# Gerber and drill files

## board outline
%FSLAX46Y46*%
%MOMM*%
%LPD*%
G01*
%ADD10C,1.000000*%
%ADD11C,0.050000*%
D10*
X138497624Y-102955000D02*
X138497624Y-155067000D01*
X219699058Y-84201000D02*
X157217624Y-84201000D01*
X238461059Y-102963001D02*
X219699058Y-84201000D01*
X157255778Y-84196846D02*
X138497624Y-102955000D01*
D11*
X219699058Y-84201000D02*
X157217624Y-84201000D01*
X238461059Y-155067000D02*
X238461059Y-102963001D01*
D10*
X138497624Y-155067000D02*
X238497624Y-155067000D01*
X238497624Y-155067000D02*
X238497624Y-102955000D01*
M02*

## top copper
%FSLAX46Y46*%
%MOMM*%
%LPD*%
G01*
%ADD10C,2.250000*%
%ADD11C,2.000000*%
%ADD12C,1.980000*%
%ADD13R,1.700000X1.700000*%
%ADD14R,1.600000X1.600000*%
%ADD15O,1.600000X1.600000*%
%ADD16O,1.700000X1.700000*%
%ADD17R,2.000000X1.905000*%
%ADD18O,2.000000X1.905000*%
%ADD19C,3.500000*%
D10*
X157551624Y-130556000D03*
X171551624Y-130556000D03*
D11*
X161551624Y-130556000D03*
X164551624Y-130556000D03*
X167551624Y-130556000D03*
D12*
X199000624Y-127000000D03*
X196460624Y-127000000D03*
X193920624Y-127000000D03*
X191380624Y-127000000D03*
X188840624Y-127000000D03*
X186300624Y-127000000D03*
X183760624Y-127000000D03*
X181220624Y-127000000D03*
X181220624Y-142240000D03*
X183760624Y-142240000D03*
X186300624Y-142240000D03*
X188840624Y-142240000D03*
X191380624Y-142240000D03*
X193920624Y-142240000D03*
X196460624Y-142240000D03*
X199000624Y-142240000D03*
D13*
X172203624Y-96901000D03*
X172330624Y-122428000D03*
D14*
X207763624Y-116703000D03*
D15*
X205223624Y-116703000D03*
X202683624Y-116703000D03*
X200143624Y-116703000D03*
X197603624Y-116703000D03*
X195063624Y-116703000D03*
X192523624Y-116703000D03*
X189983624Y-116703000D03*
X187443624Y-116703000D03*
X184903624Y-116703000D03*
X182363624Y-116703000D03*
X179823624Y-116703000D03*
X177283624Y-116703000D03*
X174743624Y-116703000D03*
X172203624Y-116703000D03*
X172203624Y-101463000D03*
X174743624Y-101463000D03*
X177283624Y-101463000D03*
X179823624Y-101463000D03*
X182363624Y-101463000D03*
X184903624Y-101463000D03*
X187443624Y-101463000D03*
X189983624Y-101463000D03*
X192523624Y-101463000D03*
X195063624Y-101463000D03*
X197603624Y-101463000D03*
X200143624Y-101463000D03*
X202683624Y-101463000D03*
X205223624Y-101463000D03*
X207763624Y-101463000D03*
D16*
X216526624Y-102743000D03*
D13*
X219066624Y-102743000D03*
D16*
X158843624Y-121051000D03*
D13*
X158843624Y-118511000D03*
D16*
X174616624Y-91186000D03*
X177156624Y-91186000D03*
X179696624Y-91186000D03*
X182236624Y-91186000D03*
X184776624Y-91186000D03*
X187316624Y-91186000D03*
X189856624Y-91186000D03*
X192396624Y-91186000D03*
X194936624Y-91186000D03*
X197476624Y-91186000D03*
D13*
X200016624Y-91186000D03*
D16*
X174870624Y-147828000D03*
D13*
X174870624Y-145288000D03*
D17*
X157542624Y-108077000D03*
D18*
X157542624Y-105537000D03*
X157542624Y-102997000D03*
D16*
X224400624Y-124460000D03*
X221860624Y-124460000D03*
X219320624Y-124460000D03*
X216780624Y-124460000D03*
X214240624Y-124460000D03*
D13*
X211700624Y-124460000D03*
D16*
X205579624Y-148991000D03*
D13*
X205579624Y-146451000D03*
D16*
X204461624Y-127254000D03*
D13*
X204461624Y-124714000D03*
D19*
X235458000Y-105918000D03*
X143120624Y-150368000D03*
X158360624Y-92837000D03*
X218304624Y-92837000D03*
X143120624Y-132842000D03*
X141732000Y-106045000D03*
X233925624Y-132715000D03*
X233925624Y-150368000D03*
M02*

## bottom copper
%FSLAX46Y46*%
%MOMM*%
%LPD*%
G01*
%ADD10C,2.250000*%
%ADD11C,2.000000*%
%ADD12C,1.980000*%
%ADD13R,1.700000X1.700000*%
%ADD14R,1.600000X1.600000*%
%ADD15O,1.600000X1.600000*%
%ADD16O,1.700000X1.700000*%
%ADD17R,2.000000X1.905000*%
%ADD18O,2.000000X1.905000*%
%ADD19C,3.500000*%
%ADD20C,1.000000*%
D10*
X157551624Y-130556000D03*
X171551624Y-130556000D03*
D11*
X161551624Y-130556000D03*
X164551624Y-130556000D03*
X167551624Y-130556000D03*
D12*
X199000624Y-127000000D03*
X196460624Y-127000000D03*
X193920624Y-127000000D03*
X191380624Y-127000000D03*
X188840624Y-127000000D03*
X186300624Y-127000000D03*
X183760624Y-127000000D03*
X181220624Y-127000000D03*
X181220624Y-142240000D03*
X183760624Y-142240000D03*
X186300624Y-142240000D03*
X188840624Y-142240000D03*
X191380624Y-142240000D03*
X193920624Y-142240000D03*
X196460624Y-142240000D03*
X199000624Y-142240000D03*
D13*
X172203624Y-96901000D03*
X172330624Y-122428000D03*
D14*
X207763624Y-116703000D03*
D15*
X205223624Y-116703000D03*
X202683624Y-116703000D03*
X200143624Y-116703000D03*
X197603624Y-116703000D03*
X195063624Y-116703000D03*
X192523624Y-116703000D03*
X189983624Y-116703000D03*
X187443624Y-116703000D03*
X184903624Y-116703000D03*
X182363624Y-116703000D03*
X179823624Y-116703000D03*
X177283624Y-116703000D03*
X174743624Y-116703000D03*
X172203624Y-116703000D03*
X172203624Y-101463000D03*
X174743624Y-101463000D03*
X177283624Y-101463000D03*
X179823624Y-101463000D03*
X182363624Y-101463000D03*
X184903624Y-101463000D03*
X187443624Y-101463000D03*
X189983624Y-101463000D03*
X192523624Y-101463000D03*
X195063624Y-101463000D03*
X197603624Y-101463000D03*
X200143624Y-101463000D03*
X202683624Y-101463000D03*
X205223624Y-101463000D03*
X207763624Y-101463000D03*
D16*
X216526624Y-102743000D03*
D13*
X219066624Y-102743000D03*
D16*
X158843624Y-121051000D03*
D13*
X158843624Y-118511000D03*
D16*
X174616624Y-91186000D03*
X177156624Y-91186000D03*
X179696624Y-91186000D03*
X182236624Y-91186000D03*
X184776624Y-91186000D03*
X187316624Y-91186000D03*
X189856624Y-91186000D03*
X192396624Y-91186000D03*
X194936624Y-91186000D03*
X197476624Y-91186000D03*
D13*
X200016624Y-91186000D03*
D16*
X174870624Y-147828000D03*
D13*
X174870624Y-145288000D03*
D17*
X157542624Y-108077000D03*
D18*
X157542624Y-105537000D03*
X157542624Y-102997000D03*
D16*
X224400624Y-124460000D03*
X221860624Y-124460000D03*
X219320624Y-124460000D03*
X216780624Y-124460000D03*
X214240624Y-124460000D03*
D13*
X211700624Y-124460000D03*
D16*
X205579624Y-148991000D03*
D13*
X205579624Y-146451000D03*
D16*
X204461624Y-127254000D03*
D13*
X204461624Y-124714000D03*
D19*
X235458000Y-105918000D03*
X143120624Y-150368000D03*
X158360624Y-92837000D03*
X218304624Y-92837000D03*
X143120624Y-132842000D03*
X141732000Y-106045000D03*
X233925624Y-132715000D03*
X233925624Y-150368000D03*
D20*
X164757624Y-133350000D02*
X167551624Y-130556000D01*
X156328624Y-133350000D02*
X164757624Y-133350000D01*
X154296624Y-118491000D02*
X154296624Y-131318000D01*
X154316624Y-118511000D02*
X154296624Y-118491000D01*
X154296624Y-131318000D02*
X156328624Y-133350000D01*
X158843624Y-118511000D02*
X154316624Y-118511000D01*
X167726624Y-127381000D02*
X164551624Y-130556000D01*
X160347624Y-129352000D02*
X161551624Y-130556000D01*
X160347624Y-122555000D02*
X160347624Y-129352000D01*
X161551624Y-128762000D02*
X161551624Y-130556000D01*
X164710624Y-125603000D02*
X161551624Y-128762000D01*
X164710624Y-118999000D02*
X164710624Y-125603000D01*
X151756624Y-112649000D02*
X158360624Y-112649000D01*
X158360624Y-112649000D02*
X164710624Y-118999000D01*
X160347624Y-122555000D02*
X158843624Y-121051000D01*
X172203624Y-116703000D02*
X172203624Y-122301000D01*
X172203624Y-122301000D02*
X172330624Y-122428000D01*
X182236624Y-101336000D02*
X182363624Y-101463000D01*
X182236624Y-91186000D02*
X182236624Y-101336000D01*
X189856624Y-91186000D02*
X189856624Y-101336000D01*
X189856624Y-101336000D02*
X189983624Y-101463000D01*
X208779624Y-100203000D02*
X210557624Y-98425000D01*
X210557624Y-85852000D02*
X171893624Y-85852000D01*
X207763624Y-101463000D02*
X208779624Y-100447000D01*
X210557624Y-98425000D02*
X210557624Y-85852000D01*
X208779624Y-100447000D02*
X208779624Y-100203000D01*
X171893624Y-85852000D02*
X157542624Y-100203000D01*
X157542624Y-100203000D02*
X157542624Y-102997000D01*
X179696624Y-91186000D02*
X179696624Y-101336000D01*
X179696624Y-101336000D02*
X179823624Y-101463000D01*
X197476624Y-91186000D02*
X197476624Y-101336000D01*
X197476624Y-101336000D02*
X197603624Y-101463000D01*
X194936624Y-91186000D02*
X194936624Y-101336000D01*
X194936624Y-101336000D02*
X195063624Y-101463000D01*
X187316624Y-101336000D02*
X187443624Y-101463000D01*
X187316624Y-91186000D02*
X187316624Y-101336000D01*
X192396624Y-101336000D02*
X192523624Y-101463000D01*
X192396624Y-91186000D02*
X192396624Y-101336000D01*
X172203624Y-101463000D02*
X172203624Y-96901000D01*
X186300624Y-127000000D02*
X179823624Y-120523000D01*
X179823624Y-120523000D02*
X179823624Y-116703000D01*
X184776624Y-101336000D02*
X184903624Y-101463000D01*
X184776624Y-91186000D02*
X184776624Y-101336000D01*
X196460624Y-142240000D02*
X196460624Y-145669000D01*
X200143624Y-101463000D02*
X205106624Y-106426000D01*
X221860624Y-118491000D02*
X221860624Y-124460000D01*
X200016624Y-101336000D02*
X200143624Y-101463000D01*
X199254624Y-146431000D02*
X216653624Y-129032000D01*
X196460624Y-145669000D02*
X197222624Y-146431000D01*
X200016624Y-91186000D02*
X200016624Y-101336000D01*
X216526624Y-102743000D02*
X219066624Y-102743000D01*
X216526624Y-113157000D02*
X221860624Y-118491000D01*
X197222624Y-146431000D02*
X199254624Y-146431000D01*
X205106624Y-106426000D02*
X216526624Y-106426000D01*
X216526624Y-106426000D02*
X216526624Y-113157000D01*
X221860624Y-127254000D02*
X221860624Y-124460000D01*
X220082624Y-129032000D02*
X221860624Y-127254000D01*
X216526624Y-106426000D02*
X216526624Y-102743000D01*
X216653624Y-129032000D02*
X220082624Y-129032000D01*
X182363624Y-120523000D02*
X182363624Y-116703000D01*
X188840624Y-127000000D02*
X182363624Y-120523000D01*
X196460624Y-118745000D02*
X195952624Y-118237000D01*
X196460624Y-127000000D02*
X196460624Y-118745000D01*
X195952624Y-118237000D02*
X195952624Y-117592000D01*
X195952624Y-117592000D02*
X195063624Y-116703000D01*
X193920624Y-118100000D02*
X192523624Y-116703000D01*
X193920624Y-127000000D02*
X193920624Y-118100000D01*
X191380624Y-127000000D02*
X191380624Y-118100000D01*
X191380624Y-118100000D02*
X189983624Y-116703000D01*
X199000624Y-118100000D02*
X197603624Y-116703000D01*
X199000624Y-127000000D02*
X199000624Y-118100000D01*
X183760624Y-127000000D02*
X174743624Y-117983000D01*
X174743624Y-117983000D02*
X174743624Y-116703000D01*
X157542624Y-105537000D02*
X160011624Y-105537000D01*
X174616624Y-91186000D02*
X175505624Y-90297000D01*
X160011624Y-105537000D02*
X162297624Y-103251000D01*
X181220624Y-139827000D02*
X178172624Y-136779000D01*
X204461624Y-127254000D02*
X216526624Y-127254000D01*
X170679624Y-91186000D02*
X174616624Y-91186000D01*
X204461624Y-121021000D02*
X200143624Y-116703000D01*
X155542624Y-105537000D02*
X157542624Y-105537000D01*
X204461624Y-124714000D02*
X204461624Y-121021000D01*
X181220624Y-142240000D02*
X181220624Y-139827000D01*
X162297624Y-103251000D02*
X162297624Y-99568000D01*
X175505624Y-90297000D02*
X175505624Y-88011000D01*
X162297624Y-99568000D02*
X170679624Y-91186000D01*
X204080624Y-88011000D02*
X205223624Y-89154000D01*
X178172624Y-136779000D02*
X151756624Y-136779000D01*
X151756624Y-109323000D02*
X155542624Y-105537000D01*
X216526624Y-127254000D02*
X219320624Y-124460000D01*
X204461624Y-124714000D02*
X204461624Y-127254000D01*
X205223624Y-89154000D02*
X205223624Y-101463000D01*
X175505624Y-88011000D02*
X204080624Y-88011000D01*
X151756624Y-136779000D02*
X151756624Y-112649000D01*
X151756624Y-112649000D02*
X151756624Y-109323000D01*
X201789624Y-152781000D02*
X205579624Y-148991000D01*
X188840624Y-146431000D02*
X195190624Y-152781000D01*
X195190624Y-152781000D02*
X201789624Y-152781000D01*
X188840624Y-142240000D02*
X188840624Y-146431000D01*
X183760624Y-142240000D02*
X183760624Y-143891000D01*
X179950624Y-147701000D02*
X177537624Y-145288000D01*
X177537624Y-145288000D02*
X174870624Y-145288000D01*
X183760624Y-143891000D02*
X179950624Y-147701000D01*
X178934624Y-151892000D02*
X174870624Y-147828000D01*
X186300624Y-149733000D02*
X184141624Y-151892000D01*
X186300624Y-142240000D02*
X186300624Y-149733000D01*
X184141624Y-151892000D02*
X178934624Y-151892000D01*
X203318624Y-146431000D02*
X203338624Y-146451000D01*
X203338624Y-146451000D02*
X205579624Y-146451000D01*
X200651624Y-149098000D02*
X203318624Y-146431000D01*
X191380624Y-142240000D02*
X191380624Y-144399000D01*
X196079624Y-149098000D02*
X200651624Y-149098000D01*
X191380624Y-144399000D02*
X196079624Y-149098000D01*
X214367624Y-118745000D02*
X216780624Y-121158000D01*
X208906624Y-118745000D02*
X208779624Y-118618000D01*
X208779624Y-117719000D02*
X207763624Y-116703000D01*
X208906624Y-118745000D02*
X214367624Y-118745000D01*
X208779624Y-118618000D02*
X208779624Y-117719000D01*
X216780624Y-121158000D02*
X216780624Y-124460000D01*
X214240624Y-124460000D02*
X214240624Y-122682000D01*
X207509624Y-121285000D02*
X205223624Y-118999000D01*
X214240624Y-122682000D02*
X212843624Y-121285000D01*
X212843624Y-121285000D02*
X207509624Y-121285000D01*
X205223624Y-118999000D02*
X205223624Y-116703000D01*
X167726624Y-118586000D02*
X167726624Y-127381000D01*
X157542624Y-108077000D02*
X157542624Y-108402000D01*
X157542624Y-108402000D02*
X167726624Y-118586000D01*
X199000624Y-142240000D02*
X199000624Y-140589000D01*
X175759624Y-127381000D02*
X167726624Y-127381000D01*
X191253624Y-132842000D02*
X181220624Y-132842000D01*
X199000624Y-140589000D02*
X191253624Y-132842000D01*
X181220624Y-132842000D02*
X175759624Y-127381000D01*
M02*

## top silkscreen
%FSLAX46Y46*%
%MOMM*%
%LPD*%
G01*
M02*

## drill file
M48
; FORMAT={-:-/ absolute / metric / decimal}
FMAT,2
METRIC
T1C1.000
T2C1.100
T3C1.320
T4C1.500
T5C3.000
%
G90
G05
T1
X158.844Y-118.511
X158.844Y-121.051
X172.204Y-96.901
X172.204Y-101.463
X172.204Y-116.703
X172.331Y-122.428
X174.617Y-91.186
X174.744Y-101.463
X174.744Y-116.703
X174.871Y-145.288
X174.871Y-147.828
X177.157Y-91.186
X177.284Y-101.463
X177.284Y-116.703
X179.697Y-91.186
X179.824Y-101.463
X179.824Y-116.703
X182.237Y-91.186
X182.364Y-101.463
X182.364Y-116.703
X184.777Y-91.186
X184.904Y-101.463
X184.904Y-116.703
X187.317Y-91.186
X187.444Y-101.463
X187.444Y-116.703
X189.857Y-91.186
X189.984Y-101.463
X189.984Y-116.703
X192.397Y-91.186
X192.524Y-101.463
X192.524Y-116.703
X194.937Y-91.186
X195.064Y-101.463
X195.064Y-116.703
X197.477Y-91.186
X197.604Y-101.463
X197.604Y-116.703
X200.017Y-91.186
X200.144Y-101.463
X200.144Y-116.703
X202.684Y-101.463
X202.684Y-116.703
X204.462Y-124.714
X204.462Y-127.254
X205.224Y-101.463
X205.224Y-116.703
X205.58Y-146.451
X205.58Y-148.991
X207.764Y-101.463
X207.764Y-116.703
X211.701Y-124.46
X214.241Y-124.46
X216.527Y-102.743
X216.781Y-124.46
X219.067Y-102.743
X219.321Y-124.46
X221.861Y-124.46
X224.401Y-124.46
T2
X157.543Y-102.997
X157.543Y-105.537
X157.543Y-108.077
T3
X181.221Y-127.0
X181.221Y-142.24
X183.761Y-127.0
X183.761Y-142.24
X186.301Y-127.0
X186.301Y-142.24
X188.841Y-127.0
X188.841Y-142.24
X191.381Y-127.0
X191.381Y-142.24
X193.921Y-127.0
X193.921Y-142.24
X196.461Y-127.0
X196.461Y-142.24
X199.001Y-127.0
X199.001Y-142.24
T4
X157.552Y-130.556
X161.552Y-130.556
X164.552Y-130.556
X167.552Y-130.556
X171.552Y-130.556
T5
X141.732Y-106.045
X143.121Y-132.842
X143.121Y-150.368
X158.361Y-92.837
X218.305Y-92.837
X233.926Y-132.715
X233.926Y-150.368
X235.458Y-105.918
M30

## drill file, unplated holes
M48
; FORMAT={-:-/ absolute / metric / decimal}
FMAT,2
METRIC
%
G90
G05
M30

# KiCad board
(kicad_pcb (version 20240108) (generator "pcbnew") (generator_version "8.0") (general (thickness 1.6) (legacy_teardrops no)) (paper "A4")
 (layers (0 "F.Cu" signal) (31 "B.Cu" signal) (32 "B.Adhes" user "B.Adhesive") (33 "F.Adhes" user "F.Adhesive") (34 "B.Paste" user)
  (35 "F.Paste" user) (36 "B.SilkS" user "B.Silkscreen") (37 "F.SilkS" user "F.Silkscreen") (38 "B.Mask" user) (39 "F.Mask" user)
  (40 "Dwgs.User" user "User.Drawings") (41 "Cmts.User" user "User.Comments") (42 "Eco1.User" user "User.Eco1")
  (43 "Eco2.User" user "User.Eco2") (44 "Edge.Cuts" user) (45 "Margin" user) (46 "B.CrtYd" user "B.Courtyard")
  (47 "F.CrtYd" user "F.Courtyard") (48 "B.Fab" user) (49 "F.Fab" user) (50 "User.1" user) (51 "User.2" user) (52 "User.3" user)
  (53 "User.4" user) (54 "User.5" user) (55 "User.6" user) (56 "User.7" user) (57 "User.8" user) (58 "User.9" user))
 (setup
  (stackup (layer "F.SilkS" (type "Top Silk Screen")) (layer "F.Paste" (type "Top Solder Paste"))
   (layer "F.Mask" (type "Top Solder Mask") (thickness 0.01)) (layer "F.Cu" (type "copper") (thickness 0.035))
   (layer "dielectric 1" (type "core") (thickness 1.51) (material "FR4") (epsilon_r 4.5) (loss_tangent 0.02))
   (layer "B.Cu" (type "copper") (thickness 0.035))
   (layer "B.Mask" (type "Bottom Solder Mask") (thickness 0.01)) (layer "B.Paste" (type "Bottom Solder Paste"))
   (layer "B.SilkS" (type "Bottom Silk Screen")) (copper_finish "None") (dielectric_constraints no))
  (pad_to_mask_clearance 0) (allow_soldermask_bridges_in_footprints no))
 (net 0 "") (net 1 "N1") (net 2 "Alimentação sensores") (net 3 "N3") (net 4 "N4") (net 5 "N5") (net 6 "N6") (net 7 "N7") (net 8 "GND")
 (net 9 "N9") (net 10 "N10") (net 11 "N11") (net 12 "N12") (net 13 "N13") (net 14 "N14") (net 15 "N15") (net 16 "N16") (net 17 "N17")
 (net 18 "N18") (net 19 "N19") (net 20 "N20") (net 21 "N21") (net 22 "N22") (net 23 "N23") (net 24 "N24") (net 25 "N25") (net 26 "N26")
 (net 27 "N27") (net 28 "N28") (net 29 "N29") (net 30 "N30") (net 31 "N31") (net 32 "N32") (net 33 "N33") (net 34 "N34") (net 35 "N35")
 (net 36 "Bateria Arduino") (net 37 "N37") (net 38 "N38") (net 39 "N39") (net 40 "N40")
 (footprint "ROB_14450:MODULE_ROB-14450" (layer "B.Cu") (at 190.110624 134.62 90)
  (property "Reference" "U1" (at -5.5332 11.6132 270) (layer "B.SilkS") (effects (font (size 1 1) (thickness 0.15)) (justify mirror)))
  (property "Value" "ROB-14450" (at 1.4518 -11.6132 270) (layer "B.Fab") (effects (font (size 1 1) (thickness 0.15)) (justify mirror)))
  (pad "1" thru_hole circle (at -7.62 8.89 90) (size 1.98 1.98) (drill 1.32) (layers "*.Cu" "*.Mask") (remove_unused_layers no) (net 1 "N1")
   (solder_mask_margin 0.102))
  (pad "2" thru_hole circle (at -7.62 6.35 90) (size 1.98 1.98) (drill 1.32) (layers "*.Cu" "*.Mask") (remove_unused_layers no)
   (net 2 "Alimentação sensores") (solder_mask_margin 0.102))
  (pad "3" thru_hole circle (at -7.62 3.81 90) (size 1.98 1.98) (drill 1.32) (layers "*.Cu" "*.Mask") (remove_unused_layers no) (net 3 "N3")
   (solder_mask_margin 0.102))
  (pad "4" thru_hole circle (at -7.62 1.27 90) (size 1.98 1.98) (drill 1.32) (layers "*.Cu" "*.Mask") (remove_unused_layers no) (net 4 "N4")
   (solder_mask_margin 0.102))
  (pad "5" thru_hole circle (at -7.62 -1.27 90) (size 1.98 1.98) (drill 1.32) (layers "*.Cu" "*.Mask") (remove_unused_layers no)
   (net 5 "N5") (solder_mask_margin 0.102))
  (pad "6" thru_hole circle (at -7.62 -3.81 90) (size 1.98 1.98) (drill 1.32) (layers "*.Cu" "*.Mask") (remove_unused_layers no)
   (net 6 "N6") (solder_mask_margin 0.102))
  (pad "7" thru_hole circle (at -7.62 -6.35 90) (size 1.98 1.98) (drill 1.32) (layers "*.Cu" "*.Mask") (remove_unused_layers no)
   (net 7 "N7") (solder_mask_margin 0.102))
  (pad "8" thru_hole circle (at -7.62 -8.89 90) (size 1.98 1.98) (drill 1.32) (layers "*.Cu" "*.Mask") (remove_unused_layers no)
   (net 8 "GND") (solder_mask_margin 0.102))
  (pad "9" thru_hole circle (at 7.62 -8.89 90) (size 1.98 1.98) (drill 1.32) (layers "*.Cu" "*.Mask") (remove_unused_layers no) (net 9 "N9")
   (solder_mask_margin 0.102))
  (pad "10" thru_hole circle (at 7.62 -6.35 90) (size 1.98 1.98) (drill 1.32) (layers "*.Cu" "*.Mask") (remove_unused_layers no)
   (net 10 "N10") (solder_mask_margin 0.102))
  (pad "11" thru_hole circle (at 7.62 -3.81 90) (size 1.98 1.98) (drill 1.32) (layers "*.Cu" "*.Mask") (remove_unused_layers no)
   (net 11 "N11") (solder_mask_margin 0.102))
  (pad "12" thru_hole circle (at 7.62 -1.27 90) (size 1.98 1.98) (drill 1.32) (layers "*.Cu" "*.Mask") (remove_unused_layers no)
   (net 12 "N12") (solder_mask_margin 0.102))
  (pad "13" thru_hole circle (at 7.62 1.27 90) (size 1.98 1.98) (drill 1.32) (layers "*.Cu" "*.Mask") (remove_unused_layers no)
   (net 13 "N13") (solder_mask_margin 0.102))
  (pad "14" thru_hole circle (at 7.62 3.81 90) (size 1.98 1.98) (drill 1.32) (layers "*.Cu" "*.Mask") (remove_unused_layers no)
   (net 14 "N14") (solder_mask_margin 0.102))
  (pad "15" thru_hole circle (at 7.62 6.35 90) (size 1.98 1.98) (drill 1.32) (layers "*.Cu" "*.Mask") (remove_unused_layers no)
   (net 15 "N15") (solder_mask_margin 0.102))
  (pad "16" thru_hole circle (at 7.62 8.89 90) (size 1.98 1.98) (drill 1.32) (layers "*.Cu" "*.Mask") (remove_unused_layers no)
   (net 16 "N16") (solder_mask_margin 0.102)))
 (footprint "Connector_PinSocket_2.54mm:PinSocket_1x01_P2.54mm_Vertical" (layer "B.Cu") (at 172.203624 96.901 180)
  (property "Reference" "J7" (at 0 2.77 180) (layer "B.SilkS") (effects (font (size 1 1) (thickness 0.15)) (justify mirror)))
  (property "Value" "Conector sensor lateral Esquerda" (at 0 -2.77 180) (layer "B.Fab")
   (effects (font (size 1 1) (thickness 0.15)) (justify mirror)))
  (pad "1" thru_hole rect (at 0 0 180) (size 1.7 1.7) (drill 1) (layers "*.Cu" "*.Mask") (remove_unused_layers no) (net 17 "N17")))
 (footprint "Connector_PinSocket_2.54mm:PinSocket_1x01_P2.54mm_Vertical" (layer "B.Cu") (at 172.330624 122.428 180)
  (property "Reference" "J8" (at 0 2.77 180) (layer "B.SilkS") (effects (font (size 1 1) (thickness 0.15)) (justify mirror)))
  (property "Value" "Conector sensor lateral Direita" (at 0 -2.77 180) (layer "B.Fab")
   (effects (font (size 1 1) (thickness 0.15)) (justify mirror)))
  (pad "1" thru_hole rect (at 0 0 180) (size 1.7 1.7) (drill 1) (layers "*.Cu" "*.Mask") (remove_unused_layers no) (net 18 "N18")))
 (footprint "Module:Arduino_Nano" (layer "B.Cu") (at 207.763624 116.703 90)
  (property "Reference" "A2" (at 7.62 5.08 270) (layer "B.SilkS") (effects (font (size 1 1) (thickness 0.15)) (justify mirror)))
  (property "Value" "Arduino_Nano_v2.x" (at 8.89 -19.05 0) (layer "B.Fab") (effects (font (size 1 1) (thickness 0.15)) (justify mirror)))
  (pad "1" thru_hole rect (at 0 0 90) (size 1.6 1.6) (drill 1) (layers "*.Cu" "*.Mask") (remove_unused_layers no) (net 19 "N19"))
  (pad "2" thru_hole oval (at 0 -2.54 90) (size 1.6 1.6) (drill 1) (layers "*.Cu" "*.Mask") (remove_unused_layers no) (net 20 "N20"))
  (pad "3" thru_hole oval (at 0 -5.08 90) (size 1.6 1.6) (drill 1) (layers "*.Cu" "*.Mask") (remove_unused_layers no) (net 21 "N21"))
  (pad "4" thru_hole oval (at 0 -7.62 90) (size 1.6 1.6) (drill 1) (layers "*.Cu" "*.Mask") (remove_unused_layers no) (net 8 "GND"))
  (pad "5" thru_hole oval (at 0 -10.16 90) (size 1.6 1.6) (drill 1) (layers "*.Cu" "*.Mask") (remove_unused_layers no) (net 16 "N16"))
  (pad "6" thru_hole oval (at 0 -12.7 90) (size 1.6 1.6) (drill 1) (layers "*.Cu" "*.Mask") (remove_unused_layers no) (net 15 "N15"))
  (pad "7" thru_hole oval (at 0 -15.24 90) (size 1.6 1.6) (drill 1) (layers "*.Cu" "*.Mask") (remove_unused_layers no) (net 14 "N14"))
  (pad "8" thru_hole oval (at 0 -17.78 90) (size 1.6 1.6) (drill 1) (layers "*.Cu" "*.Mask") (remove_unused_layers no) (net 13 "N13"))
  (pad "9" thru_hole oval (at 0 -20.32 90) (size 1.6 1.6) (drill 1) (layers "*.Cu" "*.Mask") (remove_unused_layers no) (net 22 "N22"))
  (pad "10" thru_hole oval (at 0 -22.86 90) (size 1.6 1.6) (drill 1) (layers "*.Cu" "*.Mask") (remove_unused_layers no) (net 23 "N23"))
  (pad "11" thru_hole oval (at 0 -25.4 90) (size 1.6 1.6) (drill 1) (layers "*.Cu" "*.Mask") (remove_unused_layers no) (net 12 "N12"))
  (pad "12" thru_hole oval (at 0 -27.94 90) (size 1.6 1.6) (drill 1) (layers "*.Cu" "*.Mask") (remove_unused_layers no) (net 11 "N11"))
  (pad "13" thru_hole oval (at 0 -30.48 90) (size 1.6 1.6) (drill 1) (layers "*.Cu" "*.Mask") (remove_unused_layers no) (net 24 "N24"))
  (pad "14" thru_hole oval (at 0 -33.02 90) (size 1.6 1.6) (drill 1) (layers "*.Cu" "*.Mask") (remove_unused_layers no) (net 10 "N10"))
  (pad "15" thru_hole oval (at 0 -35.56 90) (size 1.6 1.6) (drill 1) (layers "*.Cu" "*.Mask") (remove_unused_layers no) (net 18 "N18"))
  (pad "16" thru_hole oval (at 15.24 -35.56 90) (size 1.6 1.6) (drill 1) (layers "*.Cu" "*.Mask") (remove_unused_layers no) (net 17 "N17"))
  (pad "17" thru_hole oval (at 15.24 -33.02 90) (size 1.6 1.6) (drill 1) (layers "*.Cu" "*.Mask") (remove_unused_layers no) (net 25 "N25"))
  (pad "18" thru_hole oval (at 15.24 -30.48 90) (size 1.6 1.6) (drill 1) (layers "*.Cu" "*.Mask") (remove_unused_layers no) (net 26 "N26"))
  (pad "19" thru_hole oval (at 15.24 -27.94 90) (size 1.6 1.6) (drill 1) (layers "*.Cu" "*.Mask") (remove_unused_layers no) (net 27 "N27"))
  (pad "20" thru_hole oval (at 15.24 -25.4 90) (size 1.6 1.6) (drill 1) (layers "*.Cu" "*.Mask") (remove_unused_layers no) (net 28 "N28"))
  (pad "21" thru_hole oval (at 15.24 -22.86 90) (size 1.6 1.6) (drill 1) (layers "*.Cu" "*.Mask") (remove_unused_layers no) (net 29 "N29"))
  (pad "22" thru_hole oval (at 15.24 -20.32 90) (size 1.6 1.6) (drill 1) (layers "*.Cu" "*.Mask") (remove_unused_layers no) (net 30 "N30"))
  (pad "23" thru_hole oval (at 15.24 -17.78 90) (size 1.6 1.6) (drill 1) (layers "*.Cu" "*.Mask") (remove_unused_layers no) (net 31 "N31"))
  (pad "24" thru_hole oval (at 15.24 -15.24 90) (size 1.6 1.6) (drill 1) (layers "*.Cu" "*.Mask") (remove_unused_layers no) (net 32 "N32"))
  (pad "25" thru_hole oval (at 15.24 -12.7 90) (size 1.6 1.6) (drill 1) (layers "*.Cu" "*.Mask") (remove_unused_layers no) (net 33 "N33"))
  (pad "26" thru_hole oval (at 15.24 -10.16 90) (size 1.6 1.6) (drill 1) (layers "*.Cu" "*.Mask") (remove_unused_layers no) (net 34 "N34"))
  (pad "27" thru_hole oval (at 15.24 -7.62 90) (size 1.6 1.6) (drill 1) (layers "*.Cu" "*.Mask") (remove_unused_layers no)
   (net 2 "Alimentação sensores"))
  (pad "28" thru_hole oval (at 15.24 -5.08 90) (size 1.6 1.6) (drill 1) (layers "*.Cu" "*.Mask") (remove_unused_layers no) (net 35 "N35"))
  (pad "29" thru_hole oval (at 15.24 -2.54 90) (size 1.6 1.6) (drill 1) (layers "*.Cu" "*.Mask") (remove_unused_layers no) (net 8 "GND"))
  (pad "30" thru_hole oval (at 15.24 0 90) (size 1.6 1.6) (drill 1) (layers "*.Cu" "*.Mask") (remove_unused_layers no)
   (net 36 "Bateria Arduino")))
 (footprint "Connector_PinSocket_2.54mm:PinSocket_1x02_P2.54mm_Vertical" (layer "B.Cu") (at 219.066624 102.743 90)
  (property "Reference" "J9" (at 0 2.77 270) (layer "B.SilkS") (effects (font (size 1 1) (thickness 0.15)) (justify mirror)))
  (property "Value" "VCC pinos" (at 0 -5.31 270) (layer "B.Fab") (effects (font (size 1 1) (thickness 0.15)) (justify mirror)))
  (pad "1" thru_hole rect (at 0 0 90) (size 1.7 1.7) (drill 1) (layers "*.Cu" "*.Mask") (remove_unused_layers no)
   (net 2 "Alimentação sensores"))
  (pad "2" thru_hole oval (at 0 -2.54 90) (size 1.7 1.7) (drill 1) (layers "*.Cu" "*.Mask") (remove_unused_layers no)
   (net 2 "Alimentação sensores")))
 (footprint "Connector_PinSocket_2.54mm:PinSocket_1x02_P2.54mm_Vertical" (layer "B.Cu") (at 158.843624 118.511 180)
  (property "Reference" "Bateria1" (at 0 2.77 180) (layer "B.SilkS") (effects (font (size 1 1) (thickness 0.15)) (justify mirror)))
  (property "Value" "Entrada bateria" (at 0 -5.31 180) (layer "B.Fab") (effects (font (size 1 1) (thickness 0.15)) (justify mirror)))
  (pad "1" thru_hole rect (at 0 0 180) (size 1.7 1.7) (drill 1) (layers "*.Cu" "*.Mask") (remove_unused_layers no) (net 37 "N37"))
  (pad "2" thru_hole oval (at 0 -2.54 180) (size 1.7 1.7) (drill 1) (layers "*.Cu" "*.Mask") (remove_unused_layers no) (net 8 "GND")))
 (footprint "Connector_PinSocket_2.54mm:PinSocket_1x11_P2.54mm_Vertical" (layer "B.Cu") (at 200.016624 91.186 90)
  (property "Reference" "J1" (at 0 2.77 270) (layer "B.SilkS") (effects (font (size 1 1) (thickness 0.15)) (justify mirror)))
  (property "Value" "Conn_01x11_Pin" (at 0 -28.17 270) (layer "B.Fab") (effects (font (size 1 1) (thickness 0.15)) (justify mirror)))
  (pad "1" thru_hole rect (at 0 0 90) (size 1.7 1.7) (drill 1) (layers "*.Cu" "*.Mask") (remove_unused_layers no)
   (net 2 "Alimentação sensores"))
  (pad "2" thru_hole oval (at 0 -2.54 90) (size 1.7 1.7) (drill 1) (layers "*.Cu" "*.Mask") (remove_unused_layers no) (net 34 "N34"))
  (pad "3" thru_hole oval (at 0 -5.08 90) (size 1.7 1.7) (drill 1) (layers "*.Cu" "*.Mask") (remove_unused_layers no) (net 33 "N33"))
  (pad "4" thru_hole oval (at 0 -7.62 90) (size 1.7 1.7) (drill 1) (layers "*.Cu" "*.Mask") (remove_unused_layers no) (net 32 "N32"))
  (pad "5" thru_hole oval (at 0 -10.16 90) (size 1.7 1.7) (drill 1) (layers "*.Cu" "*.Mask") (remove_unused_layers no) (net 31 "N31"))
  (pad "6" thru_hole oval (at 0 -12.7 90) (size 1.7 1.7) (drill 1) (layers "*.Cu" "*.Mask") (remove_unused_layers no) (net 30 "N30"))
  (pad "7" thru_hole oval (at 0 -15.24 90) (size 1.7 1.7) (drill 1) (layers "*.Cu" "*.Mask") (remove_unused_layers no) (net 29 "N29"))
  (pad "8" thru_hole oval (at 0 -17.78 90) (size 1.7 1.7) (drill 1) (layers "*.Cu" "*.Mask") (remove_unused_layers no) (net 28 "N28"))
  (pad "9" thru_hole oval (at 0 -20.32 90) (size 1.7 1.7) (drill 1) (layers "*.Cu" "*.Mask") (remove_unused_layers no) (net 27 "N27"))
  (pad "10" thru_hole oval (at 0 -22.86 90) (size 1.7 1.7) (drill 1) (layers "*.Cu" "*.Mask") (remove_unused_layers no) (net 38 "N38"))
  (pad "11" thru_hole oval (at 0 -25.4 90) (size 1.7 1.7) (drill 1) (layers "*.Cu" "*.Mask") (remove_unused_layers no) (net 8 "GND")))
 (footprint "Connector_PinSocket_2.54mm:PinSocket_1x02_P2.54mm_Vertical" (layer "B.Cu") (at 174.870624 145.288 180)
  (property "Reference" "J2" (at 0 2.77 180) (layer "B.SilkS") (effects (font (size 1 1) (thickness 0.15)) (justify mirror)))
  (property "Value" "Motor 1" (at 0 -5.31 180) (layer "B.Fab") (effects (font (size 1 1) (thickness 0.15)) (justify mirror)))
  (pad "1" thru_hole rect (at 0 0 180) (size 1.7 1.7) (drill 1) (layers "*.Cu" "*.Mask") (remove_unused_layers no) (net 7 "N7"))
  (pad "2" thru_hole oval (at 0 -2.54 180) (size 1.7 1.7) (drill 1) (layers "*.Cu" "*.Mask") (remove_unused_layers no) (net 6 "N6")))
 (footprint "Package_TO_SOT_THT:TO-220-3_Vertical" (layer "B.Cu") (at 157.542624 108.077 90)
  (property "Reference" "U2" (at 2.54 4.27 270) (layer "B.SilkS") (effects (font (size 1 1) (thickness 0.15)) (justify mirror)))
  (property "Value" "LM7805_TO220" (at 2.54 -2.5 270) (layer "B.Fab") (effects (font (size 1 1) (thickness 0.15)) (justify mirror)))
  (pad "1" thru_hole rect (at 0 0 90) (size 1.905 2) (drill 1.1) (layers "*.Cu" "*.Mask") (remove_unused_layers no) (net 1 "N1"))
  (pad "2" thru_hole oval (at 2.54 0 90) (size 1.905 2) (drill 1.1) (layers "*.Cu" "*.Mask") (remove_unused_layers no) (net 8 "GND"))
  (pad "3" thru_hole oval (at 5.08 0 90) (size 1.905 2) (drill 1.1) (layers "*.Cu" "*.Mask") (remove_unused_layers no)
   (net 36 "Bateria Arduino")))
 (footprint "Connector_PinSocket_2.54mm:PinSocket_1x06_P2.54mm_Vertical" (layer "B.Cu") (at 211.700624 124.46 -90)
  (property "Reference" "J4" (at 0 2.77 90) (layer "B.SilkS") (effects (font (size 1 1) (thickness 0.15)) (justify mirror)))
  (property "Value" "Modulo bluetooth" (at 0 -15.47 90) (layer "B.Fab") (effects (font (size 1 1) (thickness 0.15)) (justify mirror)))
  (pad "1" thru_hole rect (at 0 0 270) (size 1.7 1.7) (drill 1) (layers "*.Cu" "*.Mask") (remove_unused_layers no) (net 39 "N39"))
  (pad "2" thru_hole oval (at 0 -2.54 270) (size 1.7 1.7) (drill 1) (layers "*.Cu" "*.Mask") (remove_unused_layers no) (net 20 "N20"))
  (pad "3" thru_hole oval (at 0 -5.08 270) (size 1.7 1.7) (drill 1) (layers "*.Cu" "*.Mask") (remove_unused_layers no) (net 19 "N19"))
  (pad "4" thru_hole oval (at 0 -7.62 270) (size 1.7 1.7) (drill 1) (layers "*.Cu" "*.Mask") (remove_unused_layers no) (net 8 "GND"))
  (pad "5" thru_hole oval (at 0 -10.16 270) (size 1.7 1.7) (drill 1) (layers "*.Cu" "*.Mask") (remove_unused_layers no)
   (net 2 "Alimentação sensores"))
  (pad "6" thru_hole oval (at 0 -12.7 270) (size 1.7 1.7) (drill 1) (layers "*.Cu" "*.Mask") (remove_unused_layers no) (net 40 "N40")))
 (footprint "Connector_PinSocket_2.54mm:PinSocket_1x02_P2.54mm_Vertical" (layer "B.Cu") (at 205.579624 146.451 180)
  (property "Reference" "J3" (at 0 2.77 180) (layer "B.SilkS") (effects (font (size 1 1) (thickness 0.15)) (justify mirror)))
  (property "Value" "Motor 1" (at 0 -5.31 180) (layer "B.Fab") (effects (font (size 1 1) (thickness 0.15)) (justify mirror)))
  (pad "1" thru_hole rect (at 0 0 180) (size 1.7 1.7) (drill 1) (layers "*.Cu" "*.Mask") (remove_unused_layers no) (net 4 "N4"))
  (pad "2" thru_hole oval (at 0 -2.54 180) (size 1.7 1.7) (drill 1) (layers "*.Cu" "*.Mask") (remove_unused_layers no) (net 5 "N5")))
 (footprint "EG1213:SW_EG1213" (layer "B.Cu") (at 164.551624 130.556 180)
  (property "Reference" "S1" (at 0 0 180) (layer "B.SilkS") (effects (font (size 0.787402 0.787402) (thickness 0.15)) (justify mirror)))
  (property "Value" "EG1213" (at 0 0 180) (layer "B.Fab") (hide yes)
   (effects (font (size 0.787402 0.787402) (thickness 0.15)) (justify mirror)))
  (pad "1" thru_hole circle (at -3 0 180) (size 2 2) (drill 1.5) (layers "*.Cu" "*.Mask") (remove_unused_layers no) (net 37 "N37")
   (solder_mask_margin 0.102) (thermal_bridge_angle 90))
  (pad "2" thru_hole circle (at 0 0 180) (size 2 2) (drill 1.5) (layers "*.Cu" "*.Mask") (remove_unused_layers no) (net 1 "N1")
   (solder_mask_margin 0.102))
  (pad "3" thru_hole circle (at 3 0 180) (size 2 2) (drill 1.5) (layers "*.Cu" "*.Mask") (remove_unused_layers no) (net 8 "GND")
   (solder_mask_margin 0.102))
  (pad "P$4" thru_hole circle (at -7 0 180) (size 2.25 2.25) (drill 1.5) (layers "*.Cu" "*.Mask") (remove_unused_layers no)
   (solder_mask_margin 0.102))
  (pad "P$5" thru_hole circle (at 7 0 180) (size 2.25 2.25) (drill 1.5) (layers "*.Cu" "*.Mask") (remove_unused_layers no)
   (solder_mask_margin 0.102)))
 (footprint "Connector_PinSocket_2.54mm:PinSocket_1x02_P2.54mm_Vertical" (layer "B.Cu") (at 204.461624 124.714 180)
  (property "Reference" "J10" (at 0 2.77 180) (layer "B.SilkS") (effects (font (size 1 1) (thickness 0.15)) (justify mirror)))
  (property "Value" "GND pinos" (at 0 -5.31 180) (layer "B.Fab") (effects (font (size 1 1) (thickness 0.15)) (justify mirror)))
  (pad "1" thru_hole rect (at 0 0 180) (size 1.7 1.7) (drill 1) (layers "*.Cu" "*.Mask") (remove_unused_layers no) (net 8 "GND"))
  (pad "2" thru_hole oval (at 0 -2.54 180) (size 1.7 1.7) (drill 1) (layers "*.Cu" "*.Mask") (remove_unused_layers no) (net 8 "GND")))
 (gr_line (start 138.497624 102.955) (end 138.497624 155.067) (stroke (width 1) (type default)) (layer "Edge.Cuts"))
 (gr_line (start 219.699058 84.201) (end 157.217624 84.201) (stroke (width 1) (type default)) (layer "Edge.Cuts"))
 (gr_line (start 238.461059 102.963001) (end 219.699058 84.201) (stroke (width 1) (type default)) (layer "Edge.Cuts"))
 (gr_line (start 157.255778 84.196846) (end 138.497624 102.955) (stroke (width 1) (type default)) (layer "Edge.Cuts"))
 (gr_line (start 219.699058 84.201) (end 157.217624 84.201) (stroke (width 0.05) (type default)) (layer "Edge.Cuts"))
 (gr_line (start 238.461059 155.067) (end 238.461059 102.963001) (stroke (width 0.05) (type default)) (layer "Edge.Cuts"))
 (gr_line (start 138.497624 155.067) (end 238.497624 155.067) (stroke (width 1) (type default)) (layer "Edge.Cuts"))
 (gr_line (start 238.497624 155.067) (end 238.497624 102.955) (stroke (width 1) (type default)) (layer "Edge.Cuts"))
 (via (at 235.458 105.918) (size 3.5) (drill 3) (layers "F.Cu" "B.Cu") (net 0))
 (via (at 143.120624 150.368) (size 3.5) (drill 3) (layers "F.Cu" "B.Cu") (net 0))
 (via (at 158.360624 92.837) (size 3.5) (drill 3) (layers "F.Cu" "B.Cu") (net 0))
 (via (at 218.304624 92.837) (size 3.5) (drill 3) (layers "F.Cu" "B.Cu") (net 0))
 (via (at 143.120624 132.842) (size 3.5) (drill 3) (layers "F.Cu" "B.Cu") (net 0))
 (via (at 141.732 106.045) (size 3.5) (drill 3) (layers "F.Cu" "B.Cu") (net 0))
 (via (at 233.925624 132.715) (size 3.5) (drill 3) (layers "F.Cu" "B.Cu") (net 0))
 (via (at 233.925624 150.368) (size 3.5) (drill 3) (layers "F.Cu" "B.Cu") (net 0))
 (segment (start 172.203624 116.703) (end 172.203624 122.301) (width 1) (layer "B.Cu") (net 18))
 (segment (start 172.203624 122.301) (end 172.330624 122.428) (width 1) (layer "B.Cu") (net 18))
 (segment (start 182.236624 101.336) (end 182.363624 101.463) (width 1) (layer "B.Cu") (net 28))
 (segment (start 182.236624 91.186) (end 182.236624 101.336) (width 1) (layer "B.Cu") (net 28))
 (segment (start 189.856624 91.186) (end 189.856624 101.336) (width 1) (layer "B.Cu") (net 31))
 (segment (start 189.856624 101.336) (end 189.983624 101.463) (width 1) (layer "B.Cu") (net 31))
 (segment (start 208.779624 100.203) (end 210.557624 98.425) (width 1) (layer "B.Cu") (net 36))
 (segment (start 210.557624 85.852) (end 171.893624 85.852) (width 1) (layer "B.Cu") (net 36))
 (segment (start 207.763624 101.463) (end 208.779624 100.447) (width 1) (layer "B.Cu") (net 36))
 (segment (start 210.557624 98.425) (end 210.557624 85.852) (width 1) (layer "B.Cu") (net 36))
 (segment (start 208.779624 100.447) (end 208.779624 100.203) (width 1) (layer "B.Cu") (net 36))
 (segment (start 171.893624 85.852) (end 157.542624 100.203) (width 1) (layer "B.Cu") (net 36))
 (segment (start 157.542624 100.203) (end 157.542624 102.997) (width 1) (layer "B.Cu") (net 36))
 (segment (start 179.696624 91.186) (end 179.696624 101.336) (width 1) (layer "B.Cu") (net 27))
 (segment (start 179.696624 101.336) (end 179.823624 101.463) (width 1) (layer "B.Cu") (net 27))
 (segment (start 197.476624 91.186) (end 197.476624 101.336) (width 1) (layer "B.Cu") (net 34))
 (segment (start 197.476624 101.336) (end 197.603624 101.463) (width 1) (layer "B.Cu") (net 34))
 (segment (start 194.936624 91.186) (end 194.936624 101.336) (width 1) (layer "B.Cu") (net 33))
 (segment (start 194.936624 101.336) (end 195.063624 101.463) (width 1) (layer "B.Cu") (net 33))
 (segment (start 187.316624 101.336) (end 187.443624 101.463) (width 1) (layer "B.Cu") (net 30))
 (segment (start 187.316624 91.186) (end 187.316624 101.336) (width 1) (layer "B.Cu") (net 30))
 (segment (start 192.396624 101.336) (end 192.523624 101.463) (width 1) (layer "B.Cu") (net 32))
 (segment (start 192.396624 91.186) (end 192.396624 101.336) (width 1) (layer "B.Cu") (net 32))
 (segment (start 172.203624 101.463) (end 172.203624 96.901) (width 1) (layer "B.Cu") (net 17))
 (segment (start 186.300624 127) (end 179.823624 120.523) (width 1) (layer "B.Cu") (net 11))
 (segment (start 179.823624 120.523) (end 179.823624 116.703) (width 1) (layer "B.Cu") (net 11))
 (segment (start 184.776624 101.336) (end 184.903624 101.463) (width 1) (layer "B.Cu") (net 29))
 (segment (start 184.776624 91.186) (end 184.776624 101.336) (width 1) (layer "B.Cu") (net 29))
 (segment (start 196.460624 142.24) (end 196.460624 145.669) (width 1) (layer "B.Cu") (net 2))
 (segment (start 200.143624 101.463) (end 205.106624 106.426) (width 1) (layer "B.Cu") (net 2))
 (segment (start 221.860624 118.491) (end 221.860624 124.46) (width 1) (layer "B.Cu") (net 2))
 (segment (start 200.016624 101.336) (end 200.143624 101.463) (width 1) (layer "B.Cu") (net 2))
 (segment (start 199.254624 146.431) (end 216.653624 129.032) (width 1) (layer "B.Cu") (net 2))
 (segment (start 196.460624 145.669) (end 197.222624 146.431) (width 1) (layer "B.Cu") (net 2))
 (segment (start 200.016624 91.186) (end 200.016624 101.336) (width 1) (layer "B.Cu") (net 2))
 (segment (start 216.526624 102.743) (end 219.066624 102.743) (width 1) (layer "B.Cu") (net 2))
 (segment (start 216.526624 113.157) (end 221.860624 118.491) (width 1) (layer "B.Cu") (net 2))
 (segment (start 197.222624 146.431) (end 199.254624 146.431) (width 1) (layer "B.Cu") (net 2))
 (segment (start 205.106624 106.426) (end 216.526624 106.426) (width 1) (layer "B.Cu") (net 2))
 (segment (start 216.526624 106.426) (end 216.526624 113.157) (width 1) (layer "B.Cu") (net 2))
 (segment (start 221.860624 127.254) (end 221.860624 124.46) (width 1) (layer "B.Cu") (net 2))
 (segment (start 220.082624 129.032) (end 221.860624 127.254) (width 1) (layer "B.Cu") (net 2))
 (segment (start 216.526624 106.426) (end 216.526624 102.743) (width 1) (layer "B.Cu") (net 2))
 (segment (start 216.653624 129.032) (end 220.082624 129.032) (width 1) (layer "B.Cu") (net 2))
 (segment (start 156.328624 133.35) (end 164.757624 133.35) (width 1) (layer "B.Cu") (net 37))
 (segment (start 158.843624 118.511) (end 154.316624 118.511) (width 1) (layer "B.Cu") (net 37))
 (segment (start 154.296624 131.318) (end 156.328624 133.35) (width 1) (layer "B.Cu") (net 37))
 (segment (start 154.296624 118.491) (end 154.296624 131.318) (width 1) (layer "B.Cu") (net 37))
 (segment (start 154.316624 118.511) (end 154.296624 118.491) (width 1) (layer "B.Cu") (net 37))
 (segment (start 164.757624 133.35) (end 167.551624 130.556) (width 1) (layer "B.Cu") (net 37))
 (segment (start 182.363624 120.523) (end 182.363624 116.703) (width 1) (layer "B.Cu") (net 12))
 (segment (start 188.840624 127) (end 182.363624 120.523) (width 1) (layer "B.Cu") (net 12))
 (segment (start 196.460624 118.745) (end 195.952624 118.237) (width 1) (layer "B.Cu") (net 15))
 (segment (start 196.460624 127) (end 196.460624 118.745) (width 1) (layer "B.Cu") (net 15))
 (segment (start 195.952624 118.237) (end 195.952624 117.592) (width 1) (layer "B.Cu") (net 15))
 (segment (start 195.952624 117.592) (end 195.063624 116.703) (width 1) (layer "B.Cu") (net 15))
 (segment (start 193.920624 118.1) (end 192.523624 116.703) (width 1) (layer "B.Cu") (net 14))
 (segment (start 193.920624 127) (end 193.920624 118.1) (width 1) (layer "B.Cu") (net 14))
 (segment (start 191.380624 127) (end 191.380624 118.1) (width 1) (layer "B.Cu") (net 13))
 (segment (start 191.380624 118.1) (end 189.983624 116.703) (width 1) (layer "B.Cu") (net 13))
 (segment (start 199.000624 118.1) (end 197.603624 116.703) (width 1) (layer "B.Cu") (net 16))
 (segment (start 199.000624 127) (end 199.000624 118.1) (width 1) (layer "B.Cu") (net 16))
 (segment (start 183.760624 127) (end 174.743624 117.983) (width 1) (layer "B.Cu") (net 10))
 (segment (start 174.743624 117.983) (end 174.743624 116.703) (width 1) (layer "B.Cu") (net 10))
 (segment (start 160.347624 129.352) (end 161.551624 130.556) (width 1) (layer "B.Cu") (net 8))
 (segment (start 160.347624 122.555) (end 160.347624 129.352) (width 1) (layer "B.Cu") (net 8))
 (segment (start 157.542624 105.537) (end 160.011624 105.537) (width 1) (layer "B.Cu") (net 8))
 (segment (start 174.616624 91.186) (end 175.505624 90.297) (width 1) (layer "B.Cu") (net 8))
 (segment (start 160.011624 105.537) (end 162.297624 103.251) (width 1) (layer "B.Cu") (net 8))
 (segment (start 181.220624 139.827) (end 178.172624 136.779) (width 1) (layer "B.Cu") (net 8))
 (segment (start 204.461624 127.254) (end 216.526624 127.254) (width 1) (layer "B.Cu") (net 8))
 (segment (start 170.679624 91.186) (end 174.616624 91.186) (width 1) (layer "B.Cu") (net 8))
 (segment (start 204.461624 121.021) (end 200.143624 116.703) (width 1) (layer "B.Cu") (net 8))
 (segment (start 155.542624 105.537) (end 157.542624 105.537) (width 1) (layer "B.Cu") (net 8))
 (segment (start 204.461624 124.714) (end 204.461624 121.021) (width 1) (layer "B.Cu") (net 8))
 (segment (start 181.220624 142.24) (end 181.220624 139.827) (width 1) (layer "B.Cu") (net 8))
 (segment (start 160.347624 122.555) (end 158.843624 121.051) (width 1) (layer "B.Cu") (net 8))
 (segment (start 162.297624 103.251) (end 162.297624 99.568) (width 1) (layer "B.Cu") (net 8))
 (segment (start 175.505624 90.297) (end 175.505624 88.011) (width 1) (layer "B.Cu") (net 8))
 (segment (start 162.297624 99.568) (end 170.679624 91.186) (width 1) (layer "B.Cu") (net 8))
 (segment (start 151.756624 112.649) (end 158.360624 112.649) (width 1) (layer "B.Cu") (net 8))
 (segment (start 204.080624 88.011) (end 205.223624 89.154) (width 1) (layer "B.Cu") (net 8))
 (segment (start 178.172624 136.779) (end 151.756624 136.779) (width 1) (layer "B.Cu") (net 8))
 (segment (start 151.756624 109.323) (end 155.542624 105.537) (width 1) (layer "B.Cu") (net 8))
 (segment (start 216.526624 127.254) (end 219.320624 124.46) (width 1) (layer "B.Cu") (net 8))
 (segment (start 204.461624 124.714) (end 204.461624 127.254) (width 1) (layer "B.Cu") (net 8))
 (segment (start 205.223624 89.154) (end 205.223624 101.463) (width 1) (layer "B.Cu") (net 8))
 (segment (start 175.505624 88.011) (end 204.080624 88.011) (width 1) (layer "B.Cu") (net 8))
 (segment (start 158.360624 112.649) (end 164.710624 118.999) (width 1) (layer "B.Cu") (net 8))
 (segment (start 161.551624 128.762) (end 161.551624 130.556) (width 1) (layer "B.Cu") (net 8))
 (segment (start 164.710624 118.999) (end 164.710624 125.603) (width 1) (layer "B.Cu") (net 8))
 (segment (start 164.710624 125.603) (end 161.551624 128.762) (width 1) (layer "B.Cu") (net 8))
 (segment (start 151.756624 136.779) (end 151.756624 112.649) (width 1) (layer "B.Cu") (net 8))
 (segment (start 151.756624 112.649) (end 151.756624 109.323) (width 1) (layer "B.Cu") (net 8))
 (segment (start 201.789624 152.781) (end 205.579624 148.991) (width 1) (layer "B.Cu") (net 5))
 (segment (start 188.840624 146.431) (end 195.190624 152.781) (width 1) (layer "B.Cu") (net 5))
 (segment (start 195.190624 152.781) (end 201.789624 152.781) (width 1) (layer "B.Cu") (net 5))
 (segment (start 188.840624 142.24) (end 188.840624 146.431) (width 1) (layer "B.Cu") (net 5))
 (segment (start 183.760624 142.24) (end 183.760624 143.891) (width 1) (layer "B.Cu") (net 7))
 (segment (start 179.950624 147.701) (end 177.537624 145.288) (width 1) (layer "B.Cu") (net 7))
 (segment (start 177.537624 145.288) (end 174.870624 145.288) (width 1) (layer "B.Cu") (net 7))
 (segment (start 183.760624 143.891) (end 179.950624 147.701) (width 1) (layer "B.Cu") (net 7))
 (segment (start 178.934624 151.892) (end 174.870624 147.828) (width 1) (layer "B.Cu") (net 6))
 (segment (start 186.300624 149.733) (end 184.141624 151.892) (width 1) (layer "B.Cu") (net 6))
 (segment (start 186.300624 142.24) (end 186.300624 149.733) (width 1) (layer "B.Cu") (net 6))
 (segment (start 184.141624 151.892) (end 178.934624 151.892) (width 1) (layer "B.Cu") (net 6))
 (segment (start 203.318624 146.431) (end 203.338624 146.451) (width 1) (layer "B.Cu") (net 4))
 (segment (start 203.338624 146.451) (end 205.579624 146.451) (width 1) (layer "B.Cu") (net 4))
 (segment (start 200.651624 149.098) (end 203.318624 146.431) (width 1) (layer "B.Cu") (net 4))
 (segment (start 191.380624 142.24) (end 191.380624 144.399) (width 1) (layer "B.Cu") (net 4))
 (segment (start 196.079624 149.098) (end 200.651624 149.098) (width 1) (layer "B.Cu") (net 4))
 (segment (start 191.380624 144.399) (end 196.079624 149.098) (width 1) (layer "B.Cu") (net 4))
 (segment (start 214.367624 118.745) (end 216.780624 121.158) (width 1) (layer "B.Cu") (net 19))
 (segment (start 208.906624 118.745) (end 208.779624 118.618) (width 1) (layer "B.Cu") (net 19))
 (segment (start 208.779624 117.719) (end 207.763624 116.703) (width 1) (layer "B.Cu") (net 19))
 (segment (start 208.906624 118.745) (end 214.367624 118.745) (width 1) (layer "B.Cu") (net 19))
 (segment (start 208.779624 118.618) (end 208.779624 117.719) (width 1) (layer "B.Cu") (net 19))
 (segment (start 216.780624 121.158) (end 216.780624 124.46) (width 1) (layer "B.Cu") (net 19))
 (segment (start 214.240624 124.46) (end 214.240624 122.682) (width 1) (layer "B.Cu") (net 20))
 (segment (start 207.509624 121.285) (end 205.223624 118.999) (width 1) (layer "B.Cu") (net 20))
 (segment (start 214.240624 122.682) (end 212.843624 121.285) (width 1) (layer "B.Cu") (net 20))
 (segment (start 212.843624 121.285) (end 207.509624 121.285) (width 1) (layer "B.Cu") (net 20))
 (segment (start 205.223624 118.999) (end 205.223624 116.703) (width 1) (layer "B.Cu") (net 20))
 (segment (start 167.726624 118.586) (end 167.726624 127.381) (width 1) (layer "B.Cu") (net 1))
 (segment (start 167.726624 127.381) (end 164.551624 130.556) (width 1) (layer "B.Cu") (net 1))
 (segment (start 157.542624 108.077) (end 157.542624 108.402) (width 1) (layer "B.Cu") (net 1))
 (segment (start 157.542624 108.402) (end 167.726624 118.586) (width 1) (layer "B.Cu") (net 1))
 (segment (start 199.000624 142.24) (end 199.000624 140.589) (width 1) (layer "B.Cu") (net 1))
 (segment (start 175.759624 127.381) (end 167.726624 127.381) (width 1) (layer "B.Cu") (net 1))
 (segment (start 191.253624 132.842) (end 181.220624 132.842) (width 1) (layer "B.Cu") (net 1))
 (segment (start 199.000624 140.589) (end 191.253624 132.842) (width 1) (layer "B.Cu") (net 1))
 (segment (start 181.220624 132.842) (end 175.759624 127.381) (width 1) (layer "B.Cu") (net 1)))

